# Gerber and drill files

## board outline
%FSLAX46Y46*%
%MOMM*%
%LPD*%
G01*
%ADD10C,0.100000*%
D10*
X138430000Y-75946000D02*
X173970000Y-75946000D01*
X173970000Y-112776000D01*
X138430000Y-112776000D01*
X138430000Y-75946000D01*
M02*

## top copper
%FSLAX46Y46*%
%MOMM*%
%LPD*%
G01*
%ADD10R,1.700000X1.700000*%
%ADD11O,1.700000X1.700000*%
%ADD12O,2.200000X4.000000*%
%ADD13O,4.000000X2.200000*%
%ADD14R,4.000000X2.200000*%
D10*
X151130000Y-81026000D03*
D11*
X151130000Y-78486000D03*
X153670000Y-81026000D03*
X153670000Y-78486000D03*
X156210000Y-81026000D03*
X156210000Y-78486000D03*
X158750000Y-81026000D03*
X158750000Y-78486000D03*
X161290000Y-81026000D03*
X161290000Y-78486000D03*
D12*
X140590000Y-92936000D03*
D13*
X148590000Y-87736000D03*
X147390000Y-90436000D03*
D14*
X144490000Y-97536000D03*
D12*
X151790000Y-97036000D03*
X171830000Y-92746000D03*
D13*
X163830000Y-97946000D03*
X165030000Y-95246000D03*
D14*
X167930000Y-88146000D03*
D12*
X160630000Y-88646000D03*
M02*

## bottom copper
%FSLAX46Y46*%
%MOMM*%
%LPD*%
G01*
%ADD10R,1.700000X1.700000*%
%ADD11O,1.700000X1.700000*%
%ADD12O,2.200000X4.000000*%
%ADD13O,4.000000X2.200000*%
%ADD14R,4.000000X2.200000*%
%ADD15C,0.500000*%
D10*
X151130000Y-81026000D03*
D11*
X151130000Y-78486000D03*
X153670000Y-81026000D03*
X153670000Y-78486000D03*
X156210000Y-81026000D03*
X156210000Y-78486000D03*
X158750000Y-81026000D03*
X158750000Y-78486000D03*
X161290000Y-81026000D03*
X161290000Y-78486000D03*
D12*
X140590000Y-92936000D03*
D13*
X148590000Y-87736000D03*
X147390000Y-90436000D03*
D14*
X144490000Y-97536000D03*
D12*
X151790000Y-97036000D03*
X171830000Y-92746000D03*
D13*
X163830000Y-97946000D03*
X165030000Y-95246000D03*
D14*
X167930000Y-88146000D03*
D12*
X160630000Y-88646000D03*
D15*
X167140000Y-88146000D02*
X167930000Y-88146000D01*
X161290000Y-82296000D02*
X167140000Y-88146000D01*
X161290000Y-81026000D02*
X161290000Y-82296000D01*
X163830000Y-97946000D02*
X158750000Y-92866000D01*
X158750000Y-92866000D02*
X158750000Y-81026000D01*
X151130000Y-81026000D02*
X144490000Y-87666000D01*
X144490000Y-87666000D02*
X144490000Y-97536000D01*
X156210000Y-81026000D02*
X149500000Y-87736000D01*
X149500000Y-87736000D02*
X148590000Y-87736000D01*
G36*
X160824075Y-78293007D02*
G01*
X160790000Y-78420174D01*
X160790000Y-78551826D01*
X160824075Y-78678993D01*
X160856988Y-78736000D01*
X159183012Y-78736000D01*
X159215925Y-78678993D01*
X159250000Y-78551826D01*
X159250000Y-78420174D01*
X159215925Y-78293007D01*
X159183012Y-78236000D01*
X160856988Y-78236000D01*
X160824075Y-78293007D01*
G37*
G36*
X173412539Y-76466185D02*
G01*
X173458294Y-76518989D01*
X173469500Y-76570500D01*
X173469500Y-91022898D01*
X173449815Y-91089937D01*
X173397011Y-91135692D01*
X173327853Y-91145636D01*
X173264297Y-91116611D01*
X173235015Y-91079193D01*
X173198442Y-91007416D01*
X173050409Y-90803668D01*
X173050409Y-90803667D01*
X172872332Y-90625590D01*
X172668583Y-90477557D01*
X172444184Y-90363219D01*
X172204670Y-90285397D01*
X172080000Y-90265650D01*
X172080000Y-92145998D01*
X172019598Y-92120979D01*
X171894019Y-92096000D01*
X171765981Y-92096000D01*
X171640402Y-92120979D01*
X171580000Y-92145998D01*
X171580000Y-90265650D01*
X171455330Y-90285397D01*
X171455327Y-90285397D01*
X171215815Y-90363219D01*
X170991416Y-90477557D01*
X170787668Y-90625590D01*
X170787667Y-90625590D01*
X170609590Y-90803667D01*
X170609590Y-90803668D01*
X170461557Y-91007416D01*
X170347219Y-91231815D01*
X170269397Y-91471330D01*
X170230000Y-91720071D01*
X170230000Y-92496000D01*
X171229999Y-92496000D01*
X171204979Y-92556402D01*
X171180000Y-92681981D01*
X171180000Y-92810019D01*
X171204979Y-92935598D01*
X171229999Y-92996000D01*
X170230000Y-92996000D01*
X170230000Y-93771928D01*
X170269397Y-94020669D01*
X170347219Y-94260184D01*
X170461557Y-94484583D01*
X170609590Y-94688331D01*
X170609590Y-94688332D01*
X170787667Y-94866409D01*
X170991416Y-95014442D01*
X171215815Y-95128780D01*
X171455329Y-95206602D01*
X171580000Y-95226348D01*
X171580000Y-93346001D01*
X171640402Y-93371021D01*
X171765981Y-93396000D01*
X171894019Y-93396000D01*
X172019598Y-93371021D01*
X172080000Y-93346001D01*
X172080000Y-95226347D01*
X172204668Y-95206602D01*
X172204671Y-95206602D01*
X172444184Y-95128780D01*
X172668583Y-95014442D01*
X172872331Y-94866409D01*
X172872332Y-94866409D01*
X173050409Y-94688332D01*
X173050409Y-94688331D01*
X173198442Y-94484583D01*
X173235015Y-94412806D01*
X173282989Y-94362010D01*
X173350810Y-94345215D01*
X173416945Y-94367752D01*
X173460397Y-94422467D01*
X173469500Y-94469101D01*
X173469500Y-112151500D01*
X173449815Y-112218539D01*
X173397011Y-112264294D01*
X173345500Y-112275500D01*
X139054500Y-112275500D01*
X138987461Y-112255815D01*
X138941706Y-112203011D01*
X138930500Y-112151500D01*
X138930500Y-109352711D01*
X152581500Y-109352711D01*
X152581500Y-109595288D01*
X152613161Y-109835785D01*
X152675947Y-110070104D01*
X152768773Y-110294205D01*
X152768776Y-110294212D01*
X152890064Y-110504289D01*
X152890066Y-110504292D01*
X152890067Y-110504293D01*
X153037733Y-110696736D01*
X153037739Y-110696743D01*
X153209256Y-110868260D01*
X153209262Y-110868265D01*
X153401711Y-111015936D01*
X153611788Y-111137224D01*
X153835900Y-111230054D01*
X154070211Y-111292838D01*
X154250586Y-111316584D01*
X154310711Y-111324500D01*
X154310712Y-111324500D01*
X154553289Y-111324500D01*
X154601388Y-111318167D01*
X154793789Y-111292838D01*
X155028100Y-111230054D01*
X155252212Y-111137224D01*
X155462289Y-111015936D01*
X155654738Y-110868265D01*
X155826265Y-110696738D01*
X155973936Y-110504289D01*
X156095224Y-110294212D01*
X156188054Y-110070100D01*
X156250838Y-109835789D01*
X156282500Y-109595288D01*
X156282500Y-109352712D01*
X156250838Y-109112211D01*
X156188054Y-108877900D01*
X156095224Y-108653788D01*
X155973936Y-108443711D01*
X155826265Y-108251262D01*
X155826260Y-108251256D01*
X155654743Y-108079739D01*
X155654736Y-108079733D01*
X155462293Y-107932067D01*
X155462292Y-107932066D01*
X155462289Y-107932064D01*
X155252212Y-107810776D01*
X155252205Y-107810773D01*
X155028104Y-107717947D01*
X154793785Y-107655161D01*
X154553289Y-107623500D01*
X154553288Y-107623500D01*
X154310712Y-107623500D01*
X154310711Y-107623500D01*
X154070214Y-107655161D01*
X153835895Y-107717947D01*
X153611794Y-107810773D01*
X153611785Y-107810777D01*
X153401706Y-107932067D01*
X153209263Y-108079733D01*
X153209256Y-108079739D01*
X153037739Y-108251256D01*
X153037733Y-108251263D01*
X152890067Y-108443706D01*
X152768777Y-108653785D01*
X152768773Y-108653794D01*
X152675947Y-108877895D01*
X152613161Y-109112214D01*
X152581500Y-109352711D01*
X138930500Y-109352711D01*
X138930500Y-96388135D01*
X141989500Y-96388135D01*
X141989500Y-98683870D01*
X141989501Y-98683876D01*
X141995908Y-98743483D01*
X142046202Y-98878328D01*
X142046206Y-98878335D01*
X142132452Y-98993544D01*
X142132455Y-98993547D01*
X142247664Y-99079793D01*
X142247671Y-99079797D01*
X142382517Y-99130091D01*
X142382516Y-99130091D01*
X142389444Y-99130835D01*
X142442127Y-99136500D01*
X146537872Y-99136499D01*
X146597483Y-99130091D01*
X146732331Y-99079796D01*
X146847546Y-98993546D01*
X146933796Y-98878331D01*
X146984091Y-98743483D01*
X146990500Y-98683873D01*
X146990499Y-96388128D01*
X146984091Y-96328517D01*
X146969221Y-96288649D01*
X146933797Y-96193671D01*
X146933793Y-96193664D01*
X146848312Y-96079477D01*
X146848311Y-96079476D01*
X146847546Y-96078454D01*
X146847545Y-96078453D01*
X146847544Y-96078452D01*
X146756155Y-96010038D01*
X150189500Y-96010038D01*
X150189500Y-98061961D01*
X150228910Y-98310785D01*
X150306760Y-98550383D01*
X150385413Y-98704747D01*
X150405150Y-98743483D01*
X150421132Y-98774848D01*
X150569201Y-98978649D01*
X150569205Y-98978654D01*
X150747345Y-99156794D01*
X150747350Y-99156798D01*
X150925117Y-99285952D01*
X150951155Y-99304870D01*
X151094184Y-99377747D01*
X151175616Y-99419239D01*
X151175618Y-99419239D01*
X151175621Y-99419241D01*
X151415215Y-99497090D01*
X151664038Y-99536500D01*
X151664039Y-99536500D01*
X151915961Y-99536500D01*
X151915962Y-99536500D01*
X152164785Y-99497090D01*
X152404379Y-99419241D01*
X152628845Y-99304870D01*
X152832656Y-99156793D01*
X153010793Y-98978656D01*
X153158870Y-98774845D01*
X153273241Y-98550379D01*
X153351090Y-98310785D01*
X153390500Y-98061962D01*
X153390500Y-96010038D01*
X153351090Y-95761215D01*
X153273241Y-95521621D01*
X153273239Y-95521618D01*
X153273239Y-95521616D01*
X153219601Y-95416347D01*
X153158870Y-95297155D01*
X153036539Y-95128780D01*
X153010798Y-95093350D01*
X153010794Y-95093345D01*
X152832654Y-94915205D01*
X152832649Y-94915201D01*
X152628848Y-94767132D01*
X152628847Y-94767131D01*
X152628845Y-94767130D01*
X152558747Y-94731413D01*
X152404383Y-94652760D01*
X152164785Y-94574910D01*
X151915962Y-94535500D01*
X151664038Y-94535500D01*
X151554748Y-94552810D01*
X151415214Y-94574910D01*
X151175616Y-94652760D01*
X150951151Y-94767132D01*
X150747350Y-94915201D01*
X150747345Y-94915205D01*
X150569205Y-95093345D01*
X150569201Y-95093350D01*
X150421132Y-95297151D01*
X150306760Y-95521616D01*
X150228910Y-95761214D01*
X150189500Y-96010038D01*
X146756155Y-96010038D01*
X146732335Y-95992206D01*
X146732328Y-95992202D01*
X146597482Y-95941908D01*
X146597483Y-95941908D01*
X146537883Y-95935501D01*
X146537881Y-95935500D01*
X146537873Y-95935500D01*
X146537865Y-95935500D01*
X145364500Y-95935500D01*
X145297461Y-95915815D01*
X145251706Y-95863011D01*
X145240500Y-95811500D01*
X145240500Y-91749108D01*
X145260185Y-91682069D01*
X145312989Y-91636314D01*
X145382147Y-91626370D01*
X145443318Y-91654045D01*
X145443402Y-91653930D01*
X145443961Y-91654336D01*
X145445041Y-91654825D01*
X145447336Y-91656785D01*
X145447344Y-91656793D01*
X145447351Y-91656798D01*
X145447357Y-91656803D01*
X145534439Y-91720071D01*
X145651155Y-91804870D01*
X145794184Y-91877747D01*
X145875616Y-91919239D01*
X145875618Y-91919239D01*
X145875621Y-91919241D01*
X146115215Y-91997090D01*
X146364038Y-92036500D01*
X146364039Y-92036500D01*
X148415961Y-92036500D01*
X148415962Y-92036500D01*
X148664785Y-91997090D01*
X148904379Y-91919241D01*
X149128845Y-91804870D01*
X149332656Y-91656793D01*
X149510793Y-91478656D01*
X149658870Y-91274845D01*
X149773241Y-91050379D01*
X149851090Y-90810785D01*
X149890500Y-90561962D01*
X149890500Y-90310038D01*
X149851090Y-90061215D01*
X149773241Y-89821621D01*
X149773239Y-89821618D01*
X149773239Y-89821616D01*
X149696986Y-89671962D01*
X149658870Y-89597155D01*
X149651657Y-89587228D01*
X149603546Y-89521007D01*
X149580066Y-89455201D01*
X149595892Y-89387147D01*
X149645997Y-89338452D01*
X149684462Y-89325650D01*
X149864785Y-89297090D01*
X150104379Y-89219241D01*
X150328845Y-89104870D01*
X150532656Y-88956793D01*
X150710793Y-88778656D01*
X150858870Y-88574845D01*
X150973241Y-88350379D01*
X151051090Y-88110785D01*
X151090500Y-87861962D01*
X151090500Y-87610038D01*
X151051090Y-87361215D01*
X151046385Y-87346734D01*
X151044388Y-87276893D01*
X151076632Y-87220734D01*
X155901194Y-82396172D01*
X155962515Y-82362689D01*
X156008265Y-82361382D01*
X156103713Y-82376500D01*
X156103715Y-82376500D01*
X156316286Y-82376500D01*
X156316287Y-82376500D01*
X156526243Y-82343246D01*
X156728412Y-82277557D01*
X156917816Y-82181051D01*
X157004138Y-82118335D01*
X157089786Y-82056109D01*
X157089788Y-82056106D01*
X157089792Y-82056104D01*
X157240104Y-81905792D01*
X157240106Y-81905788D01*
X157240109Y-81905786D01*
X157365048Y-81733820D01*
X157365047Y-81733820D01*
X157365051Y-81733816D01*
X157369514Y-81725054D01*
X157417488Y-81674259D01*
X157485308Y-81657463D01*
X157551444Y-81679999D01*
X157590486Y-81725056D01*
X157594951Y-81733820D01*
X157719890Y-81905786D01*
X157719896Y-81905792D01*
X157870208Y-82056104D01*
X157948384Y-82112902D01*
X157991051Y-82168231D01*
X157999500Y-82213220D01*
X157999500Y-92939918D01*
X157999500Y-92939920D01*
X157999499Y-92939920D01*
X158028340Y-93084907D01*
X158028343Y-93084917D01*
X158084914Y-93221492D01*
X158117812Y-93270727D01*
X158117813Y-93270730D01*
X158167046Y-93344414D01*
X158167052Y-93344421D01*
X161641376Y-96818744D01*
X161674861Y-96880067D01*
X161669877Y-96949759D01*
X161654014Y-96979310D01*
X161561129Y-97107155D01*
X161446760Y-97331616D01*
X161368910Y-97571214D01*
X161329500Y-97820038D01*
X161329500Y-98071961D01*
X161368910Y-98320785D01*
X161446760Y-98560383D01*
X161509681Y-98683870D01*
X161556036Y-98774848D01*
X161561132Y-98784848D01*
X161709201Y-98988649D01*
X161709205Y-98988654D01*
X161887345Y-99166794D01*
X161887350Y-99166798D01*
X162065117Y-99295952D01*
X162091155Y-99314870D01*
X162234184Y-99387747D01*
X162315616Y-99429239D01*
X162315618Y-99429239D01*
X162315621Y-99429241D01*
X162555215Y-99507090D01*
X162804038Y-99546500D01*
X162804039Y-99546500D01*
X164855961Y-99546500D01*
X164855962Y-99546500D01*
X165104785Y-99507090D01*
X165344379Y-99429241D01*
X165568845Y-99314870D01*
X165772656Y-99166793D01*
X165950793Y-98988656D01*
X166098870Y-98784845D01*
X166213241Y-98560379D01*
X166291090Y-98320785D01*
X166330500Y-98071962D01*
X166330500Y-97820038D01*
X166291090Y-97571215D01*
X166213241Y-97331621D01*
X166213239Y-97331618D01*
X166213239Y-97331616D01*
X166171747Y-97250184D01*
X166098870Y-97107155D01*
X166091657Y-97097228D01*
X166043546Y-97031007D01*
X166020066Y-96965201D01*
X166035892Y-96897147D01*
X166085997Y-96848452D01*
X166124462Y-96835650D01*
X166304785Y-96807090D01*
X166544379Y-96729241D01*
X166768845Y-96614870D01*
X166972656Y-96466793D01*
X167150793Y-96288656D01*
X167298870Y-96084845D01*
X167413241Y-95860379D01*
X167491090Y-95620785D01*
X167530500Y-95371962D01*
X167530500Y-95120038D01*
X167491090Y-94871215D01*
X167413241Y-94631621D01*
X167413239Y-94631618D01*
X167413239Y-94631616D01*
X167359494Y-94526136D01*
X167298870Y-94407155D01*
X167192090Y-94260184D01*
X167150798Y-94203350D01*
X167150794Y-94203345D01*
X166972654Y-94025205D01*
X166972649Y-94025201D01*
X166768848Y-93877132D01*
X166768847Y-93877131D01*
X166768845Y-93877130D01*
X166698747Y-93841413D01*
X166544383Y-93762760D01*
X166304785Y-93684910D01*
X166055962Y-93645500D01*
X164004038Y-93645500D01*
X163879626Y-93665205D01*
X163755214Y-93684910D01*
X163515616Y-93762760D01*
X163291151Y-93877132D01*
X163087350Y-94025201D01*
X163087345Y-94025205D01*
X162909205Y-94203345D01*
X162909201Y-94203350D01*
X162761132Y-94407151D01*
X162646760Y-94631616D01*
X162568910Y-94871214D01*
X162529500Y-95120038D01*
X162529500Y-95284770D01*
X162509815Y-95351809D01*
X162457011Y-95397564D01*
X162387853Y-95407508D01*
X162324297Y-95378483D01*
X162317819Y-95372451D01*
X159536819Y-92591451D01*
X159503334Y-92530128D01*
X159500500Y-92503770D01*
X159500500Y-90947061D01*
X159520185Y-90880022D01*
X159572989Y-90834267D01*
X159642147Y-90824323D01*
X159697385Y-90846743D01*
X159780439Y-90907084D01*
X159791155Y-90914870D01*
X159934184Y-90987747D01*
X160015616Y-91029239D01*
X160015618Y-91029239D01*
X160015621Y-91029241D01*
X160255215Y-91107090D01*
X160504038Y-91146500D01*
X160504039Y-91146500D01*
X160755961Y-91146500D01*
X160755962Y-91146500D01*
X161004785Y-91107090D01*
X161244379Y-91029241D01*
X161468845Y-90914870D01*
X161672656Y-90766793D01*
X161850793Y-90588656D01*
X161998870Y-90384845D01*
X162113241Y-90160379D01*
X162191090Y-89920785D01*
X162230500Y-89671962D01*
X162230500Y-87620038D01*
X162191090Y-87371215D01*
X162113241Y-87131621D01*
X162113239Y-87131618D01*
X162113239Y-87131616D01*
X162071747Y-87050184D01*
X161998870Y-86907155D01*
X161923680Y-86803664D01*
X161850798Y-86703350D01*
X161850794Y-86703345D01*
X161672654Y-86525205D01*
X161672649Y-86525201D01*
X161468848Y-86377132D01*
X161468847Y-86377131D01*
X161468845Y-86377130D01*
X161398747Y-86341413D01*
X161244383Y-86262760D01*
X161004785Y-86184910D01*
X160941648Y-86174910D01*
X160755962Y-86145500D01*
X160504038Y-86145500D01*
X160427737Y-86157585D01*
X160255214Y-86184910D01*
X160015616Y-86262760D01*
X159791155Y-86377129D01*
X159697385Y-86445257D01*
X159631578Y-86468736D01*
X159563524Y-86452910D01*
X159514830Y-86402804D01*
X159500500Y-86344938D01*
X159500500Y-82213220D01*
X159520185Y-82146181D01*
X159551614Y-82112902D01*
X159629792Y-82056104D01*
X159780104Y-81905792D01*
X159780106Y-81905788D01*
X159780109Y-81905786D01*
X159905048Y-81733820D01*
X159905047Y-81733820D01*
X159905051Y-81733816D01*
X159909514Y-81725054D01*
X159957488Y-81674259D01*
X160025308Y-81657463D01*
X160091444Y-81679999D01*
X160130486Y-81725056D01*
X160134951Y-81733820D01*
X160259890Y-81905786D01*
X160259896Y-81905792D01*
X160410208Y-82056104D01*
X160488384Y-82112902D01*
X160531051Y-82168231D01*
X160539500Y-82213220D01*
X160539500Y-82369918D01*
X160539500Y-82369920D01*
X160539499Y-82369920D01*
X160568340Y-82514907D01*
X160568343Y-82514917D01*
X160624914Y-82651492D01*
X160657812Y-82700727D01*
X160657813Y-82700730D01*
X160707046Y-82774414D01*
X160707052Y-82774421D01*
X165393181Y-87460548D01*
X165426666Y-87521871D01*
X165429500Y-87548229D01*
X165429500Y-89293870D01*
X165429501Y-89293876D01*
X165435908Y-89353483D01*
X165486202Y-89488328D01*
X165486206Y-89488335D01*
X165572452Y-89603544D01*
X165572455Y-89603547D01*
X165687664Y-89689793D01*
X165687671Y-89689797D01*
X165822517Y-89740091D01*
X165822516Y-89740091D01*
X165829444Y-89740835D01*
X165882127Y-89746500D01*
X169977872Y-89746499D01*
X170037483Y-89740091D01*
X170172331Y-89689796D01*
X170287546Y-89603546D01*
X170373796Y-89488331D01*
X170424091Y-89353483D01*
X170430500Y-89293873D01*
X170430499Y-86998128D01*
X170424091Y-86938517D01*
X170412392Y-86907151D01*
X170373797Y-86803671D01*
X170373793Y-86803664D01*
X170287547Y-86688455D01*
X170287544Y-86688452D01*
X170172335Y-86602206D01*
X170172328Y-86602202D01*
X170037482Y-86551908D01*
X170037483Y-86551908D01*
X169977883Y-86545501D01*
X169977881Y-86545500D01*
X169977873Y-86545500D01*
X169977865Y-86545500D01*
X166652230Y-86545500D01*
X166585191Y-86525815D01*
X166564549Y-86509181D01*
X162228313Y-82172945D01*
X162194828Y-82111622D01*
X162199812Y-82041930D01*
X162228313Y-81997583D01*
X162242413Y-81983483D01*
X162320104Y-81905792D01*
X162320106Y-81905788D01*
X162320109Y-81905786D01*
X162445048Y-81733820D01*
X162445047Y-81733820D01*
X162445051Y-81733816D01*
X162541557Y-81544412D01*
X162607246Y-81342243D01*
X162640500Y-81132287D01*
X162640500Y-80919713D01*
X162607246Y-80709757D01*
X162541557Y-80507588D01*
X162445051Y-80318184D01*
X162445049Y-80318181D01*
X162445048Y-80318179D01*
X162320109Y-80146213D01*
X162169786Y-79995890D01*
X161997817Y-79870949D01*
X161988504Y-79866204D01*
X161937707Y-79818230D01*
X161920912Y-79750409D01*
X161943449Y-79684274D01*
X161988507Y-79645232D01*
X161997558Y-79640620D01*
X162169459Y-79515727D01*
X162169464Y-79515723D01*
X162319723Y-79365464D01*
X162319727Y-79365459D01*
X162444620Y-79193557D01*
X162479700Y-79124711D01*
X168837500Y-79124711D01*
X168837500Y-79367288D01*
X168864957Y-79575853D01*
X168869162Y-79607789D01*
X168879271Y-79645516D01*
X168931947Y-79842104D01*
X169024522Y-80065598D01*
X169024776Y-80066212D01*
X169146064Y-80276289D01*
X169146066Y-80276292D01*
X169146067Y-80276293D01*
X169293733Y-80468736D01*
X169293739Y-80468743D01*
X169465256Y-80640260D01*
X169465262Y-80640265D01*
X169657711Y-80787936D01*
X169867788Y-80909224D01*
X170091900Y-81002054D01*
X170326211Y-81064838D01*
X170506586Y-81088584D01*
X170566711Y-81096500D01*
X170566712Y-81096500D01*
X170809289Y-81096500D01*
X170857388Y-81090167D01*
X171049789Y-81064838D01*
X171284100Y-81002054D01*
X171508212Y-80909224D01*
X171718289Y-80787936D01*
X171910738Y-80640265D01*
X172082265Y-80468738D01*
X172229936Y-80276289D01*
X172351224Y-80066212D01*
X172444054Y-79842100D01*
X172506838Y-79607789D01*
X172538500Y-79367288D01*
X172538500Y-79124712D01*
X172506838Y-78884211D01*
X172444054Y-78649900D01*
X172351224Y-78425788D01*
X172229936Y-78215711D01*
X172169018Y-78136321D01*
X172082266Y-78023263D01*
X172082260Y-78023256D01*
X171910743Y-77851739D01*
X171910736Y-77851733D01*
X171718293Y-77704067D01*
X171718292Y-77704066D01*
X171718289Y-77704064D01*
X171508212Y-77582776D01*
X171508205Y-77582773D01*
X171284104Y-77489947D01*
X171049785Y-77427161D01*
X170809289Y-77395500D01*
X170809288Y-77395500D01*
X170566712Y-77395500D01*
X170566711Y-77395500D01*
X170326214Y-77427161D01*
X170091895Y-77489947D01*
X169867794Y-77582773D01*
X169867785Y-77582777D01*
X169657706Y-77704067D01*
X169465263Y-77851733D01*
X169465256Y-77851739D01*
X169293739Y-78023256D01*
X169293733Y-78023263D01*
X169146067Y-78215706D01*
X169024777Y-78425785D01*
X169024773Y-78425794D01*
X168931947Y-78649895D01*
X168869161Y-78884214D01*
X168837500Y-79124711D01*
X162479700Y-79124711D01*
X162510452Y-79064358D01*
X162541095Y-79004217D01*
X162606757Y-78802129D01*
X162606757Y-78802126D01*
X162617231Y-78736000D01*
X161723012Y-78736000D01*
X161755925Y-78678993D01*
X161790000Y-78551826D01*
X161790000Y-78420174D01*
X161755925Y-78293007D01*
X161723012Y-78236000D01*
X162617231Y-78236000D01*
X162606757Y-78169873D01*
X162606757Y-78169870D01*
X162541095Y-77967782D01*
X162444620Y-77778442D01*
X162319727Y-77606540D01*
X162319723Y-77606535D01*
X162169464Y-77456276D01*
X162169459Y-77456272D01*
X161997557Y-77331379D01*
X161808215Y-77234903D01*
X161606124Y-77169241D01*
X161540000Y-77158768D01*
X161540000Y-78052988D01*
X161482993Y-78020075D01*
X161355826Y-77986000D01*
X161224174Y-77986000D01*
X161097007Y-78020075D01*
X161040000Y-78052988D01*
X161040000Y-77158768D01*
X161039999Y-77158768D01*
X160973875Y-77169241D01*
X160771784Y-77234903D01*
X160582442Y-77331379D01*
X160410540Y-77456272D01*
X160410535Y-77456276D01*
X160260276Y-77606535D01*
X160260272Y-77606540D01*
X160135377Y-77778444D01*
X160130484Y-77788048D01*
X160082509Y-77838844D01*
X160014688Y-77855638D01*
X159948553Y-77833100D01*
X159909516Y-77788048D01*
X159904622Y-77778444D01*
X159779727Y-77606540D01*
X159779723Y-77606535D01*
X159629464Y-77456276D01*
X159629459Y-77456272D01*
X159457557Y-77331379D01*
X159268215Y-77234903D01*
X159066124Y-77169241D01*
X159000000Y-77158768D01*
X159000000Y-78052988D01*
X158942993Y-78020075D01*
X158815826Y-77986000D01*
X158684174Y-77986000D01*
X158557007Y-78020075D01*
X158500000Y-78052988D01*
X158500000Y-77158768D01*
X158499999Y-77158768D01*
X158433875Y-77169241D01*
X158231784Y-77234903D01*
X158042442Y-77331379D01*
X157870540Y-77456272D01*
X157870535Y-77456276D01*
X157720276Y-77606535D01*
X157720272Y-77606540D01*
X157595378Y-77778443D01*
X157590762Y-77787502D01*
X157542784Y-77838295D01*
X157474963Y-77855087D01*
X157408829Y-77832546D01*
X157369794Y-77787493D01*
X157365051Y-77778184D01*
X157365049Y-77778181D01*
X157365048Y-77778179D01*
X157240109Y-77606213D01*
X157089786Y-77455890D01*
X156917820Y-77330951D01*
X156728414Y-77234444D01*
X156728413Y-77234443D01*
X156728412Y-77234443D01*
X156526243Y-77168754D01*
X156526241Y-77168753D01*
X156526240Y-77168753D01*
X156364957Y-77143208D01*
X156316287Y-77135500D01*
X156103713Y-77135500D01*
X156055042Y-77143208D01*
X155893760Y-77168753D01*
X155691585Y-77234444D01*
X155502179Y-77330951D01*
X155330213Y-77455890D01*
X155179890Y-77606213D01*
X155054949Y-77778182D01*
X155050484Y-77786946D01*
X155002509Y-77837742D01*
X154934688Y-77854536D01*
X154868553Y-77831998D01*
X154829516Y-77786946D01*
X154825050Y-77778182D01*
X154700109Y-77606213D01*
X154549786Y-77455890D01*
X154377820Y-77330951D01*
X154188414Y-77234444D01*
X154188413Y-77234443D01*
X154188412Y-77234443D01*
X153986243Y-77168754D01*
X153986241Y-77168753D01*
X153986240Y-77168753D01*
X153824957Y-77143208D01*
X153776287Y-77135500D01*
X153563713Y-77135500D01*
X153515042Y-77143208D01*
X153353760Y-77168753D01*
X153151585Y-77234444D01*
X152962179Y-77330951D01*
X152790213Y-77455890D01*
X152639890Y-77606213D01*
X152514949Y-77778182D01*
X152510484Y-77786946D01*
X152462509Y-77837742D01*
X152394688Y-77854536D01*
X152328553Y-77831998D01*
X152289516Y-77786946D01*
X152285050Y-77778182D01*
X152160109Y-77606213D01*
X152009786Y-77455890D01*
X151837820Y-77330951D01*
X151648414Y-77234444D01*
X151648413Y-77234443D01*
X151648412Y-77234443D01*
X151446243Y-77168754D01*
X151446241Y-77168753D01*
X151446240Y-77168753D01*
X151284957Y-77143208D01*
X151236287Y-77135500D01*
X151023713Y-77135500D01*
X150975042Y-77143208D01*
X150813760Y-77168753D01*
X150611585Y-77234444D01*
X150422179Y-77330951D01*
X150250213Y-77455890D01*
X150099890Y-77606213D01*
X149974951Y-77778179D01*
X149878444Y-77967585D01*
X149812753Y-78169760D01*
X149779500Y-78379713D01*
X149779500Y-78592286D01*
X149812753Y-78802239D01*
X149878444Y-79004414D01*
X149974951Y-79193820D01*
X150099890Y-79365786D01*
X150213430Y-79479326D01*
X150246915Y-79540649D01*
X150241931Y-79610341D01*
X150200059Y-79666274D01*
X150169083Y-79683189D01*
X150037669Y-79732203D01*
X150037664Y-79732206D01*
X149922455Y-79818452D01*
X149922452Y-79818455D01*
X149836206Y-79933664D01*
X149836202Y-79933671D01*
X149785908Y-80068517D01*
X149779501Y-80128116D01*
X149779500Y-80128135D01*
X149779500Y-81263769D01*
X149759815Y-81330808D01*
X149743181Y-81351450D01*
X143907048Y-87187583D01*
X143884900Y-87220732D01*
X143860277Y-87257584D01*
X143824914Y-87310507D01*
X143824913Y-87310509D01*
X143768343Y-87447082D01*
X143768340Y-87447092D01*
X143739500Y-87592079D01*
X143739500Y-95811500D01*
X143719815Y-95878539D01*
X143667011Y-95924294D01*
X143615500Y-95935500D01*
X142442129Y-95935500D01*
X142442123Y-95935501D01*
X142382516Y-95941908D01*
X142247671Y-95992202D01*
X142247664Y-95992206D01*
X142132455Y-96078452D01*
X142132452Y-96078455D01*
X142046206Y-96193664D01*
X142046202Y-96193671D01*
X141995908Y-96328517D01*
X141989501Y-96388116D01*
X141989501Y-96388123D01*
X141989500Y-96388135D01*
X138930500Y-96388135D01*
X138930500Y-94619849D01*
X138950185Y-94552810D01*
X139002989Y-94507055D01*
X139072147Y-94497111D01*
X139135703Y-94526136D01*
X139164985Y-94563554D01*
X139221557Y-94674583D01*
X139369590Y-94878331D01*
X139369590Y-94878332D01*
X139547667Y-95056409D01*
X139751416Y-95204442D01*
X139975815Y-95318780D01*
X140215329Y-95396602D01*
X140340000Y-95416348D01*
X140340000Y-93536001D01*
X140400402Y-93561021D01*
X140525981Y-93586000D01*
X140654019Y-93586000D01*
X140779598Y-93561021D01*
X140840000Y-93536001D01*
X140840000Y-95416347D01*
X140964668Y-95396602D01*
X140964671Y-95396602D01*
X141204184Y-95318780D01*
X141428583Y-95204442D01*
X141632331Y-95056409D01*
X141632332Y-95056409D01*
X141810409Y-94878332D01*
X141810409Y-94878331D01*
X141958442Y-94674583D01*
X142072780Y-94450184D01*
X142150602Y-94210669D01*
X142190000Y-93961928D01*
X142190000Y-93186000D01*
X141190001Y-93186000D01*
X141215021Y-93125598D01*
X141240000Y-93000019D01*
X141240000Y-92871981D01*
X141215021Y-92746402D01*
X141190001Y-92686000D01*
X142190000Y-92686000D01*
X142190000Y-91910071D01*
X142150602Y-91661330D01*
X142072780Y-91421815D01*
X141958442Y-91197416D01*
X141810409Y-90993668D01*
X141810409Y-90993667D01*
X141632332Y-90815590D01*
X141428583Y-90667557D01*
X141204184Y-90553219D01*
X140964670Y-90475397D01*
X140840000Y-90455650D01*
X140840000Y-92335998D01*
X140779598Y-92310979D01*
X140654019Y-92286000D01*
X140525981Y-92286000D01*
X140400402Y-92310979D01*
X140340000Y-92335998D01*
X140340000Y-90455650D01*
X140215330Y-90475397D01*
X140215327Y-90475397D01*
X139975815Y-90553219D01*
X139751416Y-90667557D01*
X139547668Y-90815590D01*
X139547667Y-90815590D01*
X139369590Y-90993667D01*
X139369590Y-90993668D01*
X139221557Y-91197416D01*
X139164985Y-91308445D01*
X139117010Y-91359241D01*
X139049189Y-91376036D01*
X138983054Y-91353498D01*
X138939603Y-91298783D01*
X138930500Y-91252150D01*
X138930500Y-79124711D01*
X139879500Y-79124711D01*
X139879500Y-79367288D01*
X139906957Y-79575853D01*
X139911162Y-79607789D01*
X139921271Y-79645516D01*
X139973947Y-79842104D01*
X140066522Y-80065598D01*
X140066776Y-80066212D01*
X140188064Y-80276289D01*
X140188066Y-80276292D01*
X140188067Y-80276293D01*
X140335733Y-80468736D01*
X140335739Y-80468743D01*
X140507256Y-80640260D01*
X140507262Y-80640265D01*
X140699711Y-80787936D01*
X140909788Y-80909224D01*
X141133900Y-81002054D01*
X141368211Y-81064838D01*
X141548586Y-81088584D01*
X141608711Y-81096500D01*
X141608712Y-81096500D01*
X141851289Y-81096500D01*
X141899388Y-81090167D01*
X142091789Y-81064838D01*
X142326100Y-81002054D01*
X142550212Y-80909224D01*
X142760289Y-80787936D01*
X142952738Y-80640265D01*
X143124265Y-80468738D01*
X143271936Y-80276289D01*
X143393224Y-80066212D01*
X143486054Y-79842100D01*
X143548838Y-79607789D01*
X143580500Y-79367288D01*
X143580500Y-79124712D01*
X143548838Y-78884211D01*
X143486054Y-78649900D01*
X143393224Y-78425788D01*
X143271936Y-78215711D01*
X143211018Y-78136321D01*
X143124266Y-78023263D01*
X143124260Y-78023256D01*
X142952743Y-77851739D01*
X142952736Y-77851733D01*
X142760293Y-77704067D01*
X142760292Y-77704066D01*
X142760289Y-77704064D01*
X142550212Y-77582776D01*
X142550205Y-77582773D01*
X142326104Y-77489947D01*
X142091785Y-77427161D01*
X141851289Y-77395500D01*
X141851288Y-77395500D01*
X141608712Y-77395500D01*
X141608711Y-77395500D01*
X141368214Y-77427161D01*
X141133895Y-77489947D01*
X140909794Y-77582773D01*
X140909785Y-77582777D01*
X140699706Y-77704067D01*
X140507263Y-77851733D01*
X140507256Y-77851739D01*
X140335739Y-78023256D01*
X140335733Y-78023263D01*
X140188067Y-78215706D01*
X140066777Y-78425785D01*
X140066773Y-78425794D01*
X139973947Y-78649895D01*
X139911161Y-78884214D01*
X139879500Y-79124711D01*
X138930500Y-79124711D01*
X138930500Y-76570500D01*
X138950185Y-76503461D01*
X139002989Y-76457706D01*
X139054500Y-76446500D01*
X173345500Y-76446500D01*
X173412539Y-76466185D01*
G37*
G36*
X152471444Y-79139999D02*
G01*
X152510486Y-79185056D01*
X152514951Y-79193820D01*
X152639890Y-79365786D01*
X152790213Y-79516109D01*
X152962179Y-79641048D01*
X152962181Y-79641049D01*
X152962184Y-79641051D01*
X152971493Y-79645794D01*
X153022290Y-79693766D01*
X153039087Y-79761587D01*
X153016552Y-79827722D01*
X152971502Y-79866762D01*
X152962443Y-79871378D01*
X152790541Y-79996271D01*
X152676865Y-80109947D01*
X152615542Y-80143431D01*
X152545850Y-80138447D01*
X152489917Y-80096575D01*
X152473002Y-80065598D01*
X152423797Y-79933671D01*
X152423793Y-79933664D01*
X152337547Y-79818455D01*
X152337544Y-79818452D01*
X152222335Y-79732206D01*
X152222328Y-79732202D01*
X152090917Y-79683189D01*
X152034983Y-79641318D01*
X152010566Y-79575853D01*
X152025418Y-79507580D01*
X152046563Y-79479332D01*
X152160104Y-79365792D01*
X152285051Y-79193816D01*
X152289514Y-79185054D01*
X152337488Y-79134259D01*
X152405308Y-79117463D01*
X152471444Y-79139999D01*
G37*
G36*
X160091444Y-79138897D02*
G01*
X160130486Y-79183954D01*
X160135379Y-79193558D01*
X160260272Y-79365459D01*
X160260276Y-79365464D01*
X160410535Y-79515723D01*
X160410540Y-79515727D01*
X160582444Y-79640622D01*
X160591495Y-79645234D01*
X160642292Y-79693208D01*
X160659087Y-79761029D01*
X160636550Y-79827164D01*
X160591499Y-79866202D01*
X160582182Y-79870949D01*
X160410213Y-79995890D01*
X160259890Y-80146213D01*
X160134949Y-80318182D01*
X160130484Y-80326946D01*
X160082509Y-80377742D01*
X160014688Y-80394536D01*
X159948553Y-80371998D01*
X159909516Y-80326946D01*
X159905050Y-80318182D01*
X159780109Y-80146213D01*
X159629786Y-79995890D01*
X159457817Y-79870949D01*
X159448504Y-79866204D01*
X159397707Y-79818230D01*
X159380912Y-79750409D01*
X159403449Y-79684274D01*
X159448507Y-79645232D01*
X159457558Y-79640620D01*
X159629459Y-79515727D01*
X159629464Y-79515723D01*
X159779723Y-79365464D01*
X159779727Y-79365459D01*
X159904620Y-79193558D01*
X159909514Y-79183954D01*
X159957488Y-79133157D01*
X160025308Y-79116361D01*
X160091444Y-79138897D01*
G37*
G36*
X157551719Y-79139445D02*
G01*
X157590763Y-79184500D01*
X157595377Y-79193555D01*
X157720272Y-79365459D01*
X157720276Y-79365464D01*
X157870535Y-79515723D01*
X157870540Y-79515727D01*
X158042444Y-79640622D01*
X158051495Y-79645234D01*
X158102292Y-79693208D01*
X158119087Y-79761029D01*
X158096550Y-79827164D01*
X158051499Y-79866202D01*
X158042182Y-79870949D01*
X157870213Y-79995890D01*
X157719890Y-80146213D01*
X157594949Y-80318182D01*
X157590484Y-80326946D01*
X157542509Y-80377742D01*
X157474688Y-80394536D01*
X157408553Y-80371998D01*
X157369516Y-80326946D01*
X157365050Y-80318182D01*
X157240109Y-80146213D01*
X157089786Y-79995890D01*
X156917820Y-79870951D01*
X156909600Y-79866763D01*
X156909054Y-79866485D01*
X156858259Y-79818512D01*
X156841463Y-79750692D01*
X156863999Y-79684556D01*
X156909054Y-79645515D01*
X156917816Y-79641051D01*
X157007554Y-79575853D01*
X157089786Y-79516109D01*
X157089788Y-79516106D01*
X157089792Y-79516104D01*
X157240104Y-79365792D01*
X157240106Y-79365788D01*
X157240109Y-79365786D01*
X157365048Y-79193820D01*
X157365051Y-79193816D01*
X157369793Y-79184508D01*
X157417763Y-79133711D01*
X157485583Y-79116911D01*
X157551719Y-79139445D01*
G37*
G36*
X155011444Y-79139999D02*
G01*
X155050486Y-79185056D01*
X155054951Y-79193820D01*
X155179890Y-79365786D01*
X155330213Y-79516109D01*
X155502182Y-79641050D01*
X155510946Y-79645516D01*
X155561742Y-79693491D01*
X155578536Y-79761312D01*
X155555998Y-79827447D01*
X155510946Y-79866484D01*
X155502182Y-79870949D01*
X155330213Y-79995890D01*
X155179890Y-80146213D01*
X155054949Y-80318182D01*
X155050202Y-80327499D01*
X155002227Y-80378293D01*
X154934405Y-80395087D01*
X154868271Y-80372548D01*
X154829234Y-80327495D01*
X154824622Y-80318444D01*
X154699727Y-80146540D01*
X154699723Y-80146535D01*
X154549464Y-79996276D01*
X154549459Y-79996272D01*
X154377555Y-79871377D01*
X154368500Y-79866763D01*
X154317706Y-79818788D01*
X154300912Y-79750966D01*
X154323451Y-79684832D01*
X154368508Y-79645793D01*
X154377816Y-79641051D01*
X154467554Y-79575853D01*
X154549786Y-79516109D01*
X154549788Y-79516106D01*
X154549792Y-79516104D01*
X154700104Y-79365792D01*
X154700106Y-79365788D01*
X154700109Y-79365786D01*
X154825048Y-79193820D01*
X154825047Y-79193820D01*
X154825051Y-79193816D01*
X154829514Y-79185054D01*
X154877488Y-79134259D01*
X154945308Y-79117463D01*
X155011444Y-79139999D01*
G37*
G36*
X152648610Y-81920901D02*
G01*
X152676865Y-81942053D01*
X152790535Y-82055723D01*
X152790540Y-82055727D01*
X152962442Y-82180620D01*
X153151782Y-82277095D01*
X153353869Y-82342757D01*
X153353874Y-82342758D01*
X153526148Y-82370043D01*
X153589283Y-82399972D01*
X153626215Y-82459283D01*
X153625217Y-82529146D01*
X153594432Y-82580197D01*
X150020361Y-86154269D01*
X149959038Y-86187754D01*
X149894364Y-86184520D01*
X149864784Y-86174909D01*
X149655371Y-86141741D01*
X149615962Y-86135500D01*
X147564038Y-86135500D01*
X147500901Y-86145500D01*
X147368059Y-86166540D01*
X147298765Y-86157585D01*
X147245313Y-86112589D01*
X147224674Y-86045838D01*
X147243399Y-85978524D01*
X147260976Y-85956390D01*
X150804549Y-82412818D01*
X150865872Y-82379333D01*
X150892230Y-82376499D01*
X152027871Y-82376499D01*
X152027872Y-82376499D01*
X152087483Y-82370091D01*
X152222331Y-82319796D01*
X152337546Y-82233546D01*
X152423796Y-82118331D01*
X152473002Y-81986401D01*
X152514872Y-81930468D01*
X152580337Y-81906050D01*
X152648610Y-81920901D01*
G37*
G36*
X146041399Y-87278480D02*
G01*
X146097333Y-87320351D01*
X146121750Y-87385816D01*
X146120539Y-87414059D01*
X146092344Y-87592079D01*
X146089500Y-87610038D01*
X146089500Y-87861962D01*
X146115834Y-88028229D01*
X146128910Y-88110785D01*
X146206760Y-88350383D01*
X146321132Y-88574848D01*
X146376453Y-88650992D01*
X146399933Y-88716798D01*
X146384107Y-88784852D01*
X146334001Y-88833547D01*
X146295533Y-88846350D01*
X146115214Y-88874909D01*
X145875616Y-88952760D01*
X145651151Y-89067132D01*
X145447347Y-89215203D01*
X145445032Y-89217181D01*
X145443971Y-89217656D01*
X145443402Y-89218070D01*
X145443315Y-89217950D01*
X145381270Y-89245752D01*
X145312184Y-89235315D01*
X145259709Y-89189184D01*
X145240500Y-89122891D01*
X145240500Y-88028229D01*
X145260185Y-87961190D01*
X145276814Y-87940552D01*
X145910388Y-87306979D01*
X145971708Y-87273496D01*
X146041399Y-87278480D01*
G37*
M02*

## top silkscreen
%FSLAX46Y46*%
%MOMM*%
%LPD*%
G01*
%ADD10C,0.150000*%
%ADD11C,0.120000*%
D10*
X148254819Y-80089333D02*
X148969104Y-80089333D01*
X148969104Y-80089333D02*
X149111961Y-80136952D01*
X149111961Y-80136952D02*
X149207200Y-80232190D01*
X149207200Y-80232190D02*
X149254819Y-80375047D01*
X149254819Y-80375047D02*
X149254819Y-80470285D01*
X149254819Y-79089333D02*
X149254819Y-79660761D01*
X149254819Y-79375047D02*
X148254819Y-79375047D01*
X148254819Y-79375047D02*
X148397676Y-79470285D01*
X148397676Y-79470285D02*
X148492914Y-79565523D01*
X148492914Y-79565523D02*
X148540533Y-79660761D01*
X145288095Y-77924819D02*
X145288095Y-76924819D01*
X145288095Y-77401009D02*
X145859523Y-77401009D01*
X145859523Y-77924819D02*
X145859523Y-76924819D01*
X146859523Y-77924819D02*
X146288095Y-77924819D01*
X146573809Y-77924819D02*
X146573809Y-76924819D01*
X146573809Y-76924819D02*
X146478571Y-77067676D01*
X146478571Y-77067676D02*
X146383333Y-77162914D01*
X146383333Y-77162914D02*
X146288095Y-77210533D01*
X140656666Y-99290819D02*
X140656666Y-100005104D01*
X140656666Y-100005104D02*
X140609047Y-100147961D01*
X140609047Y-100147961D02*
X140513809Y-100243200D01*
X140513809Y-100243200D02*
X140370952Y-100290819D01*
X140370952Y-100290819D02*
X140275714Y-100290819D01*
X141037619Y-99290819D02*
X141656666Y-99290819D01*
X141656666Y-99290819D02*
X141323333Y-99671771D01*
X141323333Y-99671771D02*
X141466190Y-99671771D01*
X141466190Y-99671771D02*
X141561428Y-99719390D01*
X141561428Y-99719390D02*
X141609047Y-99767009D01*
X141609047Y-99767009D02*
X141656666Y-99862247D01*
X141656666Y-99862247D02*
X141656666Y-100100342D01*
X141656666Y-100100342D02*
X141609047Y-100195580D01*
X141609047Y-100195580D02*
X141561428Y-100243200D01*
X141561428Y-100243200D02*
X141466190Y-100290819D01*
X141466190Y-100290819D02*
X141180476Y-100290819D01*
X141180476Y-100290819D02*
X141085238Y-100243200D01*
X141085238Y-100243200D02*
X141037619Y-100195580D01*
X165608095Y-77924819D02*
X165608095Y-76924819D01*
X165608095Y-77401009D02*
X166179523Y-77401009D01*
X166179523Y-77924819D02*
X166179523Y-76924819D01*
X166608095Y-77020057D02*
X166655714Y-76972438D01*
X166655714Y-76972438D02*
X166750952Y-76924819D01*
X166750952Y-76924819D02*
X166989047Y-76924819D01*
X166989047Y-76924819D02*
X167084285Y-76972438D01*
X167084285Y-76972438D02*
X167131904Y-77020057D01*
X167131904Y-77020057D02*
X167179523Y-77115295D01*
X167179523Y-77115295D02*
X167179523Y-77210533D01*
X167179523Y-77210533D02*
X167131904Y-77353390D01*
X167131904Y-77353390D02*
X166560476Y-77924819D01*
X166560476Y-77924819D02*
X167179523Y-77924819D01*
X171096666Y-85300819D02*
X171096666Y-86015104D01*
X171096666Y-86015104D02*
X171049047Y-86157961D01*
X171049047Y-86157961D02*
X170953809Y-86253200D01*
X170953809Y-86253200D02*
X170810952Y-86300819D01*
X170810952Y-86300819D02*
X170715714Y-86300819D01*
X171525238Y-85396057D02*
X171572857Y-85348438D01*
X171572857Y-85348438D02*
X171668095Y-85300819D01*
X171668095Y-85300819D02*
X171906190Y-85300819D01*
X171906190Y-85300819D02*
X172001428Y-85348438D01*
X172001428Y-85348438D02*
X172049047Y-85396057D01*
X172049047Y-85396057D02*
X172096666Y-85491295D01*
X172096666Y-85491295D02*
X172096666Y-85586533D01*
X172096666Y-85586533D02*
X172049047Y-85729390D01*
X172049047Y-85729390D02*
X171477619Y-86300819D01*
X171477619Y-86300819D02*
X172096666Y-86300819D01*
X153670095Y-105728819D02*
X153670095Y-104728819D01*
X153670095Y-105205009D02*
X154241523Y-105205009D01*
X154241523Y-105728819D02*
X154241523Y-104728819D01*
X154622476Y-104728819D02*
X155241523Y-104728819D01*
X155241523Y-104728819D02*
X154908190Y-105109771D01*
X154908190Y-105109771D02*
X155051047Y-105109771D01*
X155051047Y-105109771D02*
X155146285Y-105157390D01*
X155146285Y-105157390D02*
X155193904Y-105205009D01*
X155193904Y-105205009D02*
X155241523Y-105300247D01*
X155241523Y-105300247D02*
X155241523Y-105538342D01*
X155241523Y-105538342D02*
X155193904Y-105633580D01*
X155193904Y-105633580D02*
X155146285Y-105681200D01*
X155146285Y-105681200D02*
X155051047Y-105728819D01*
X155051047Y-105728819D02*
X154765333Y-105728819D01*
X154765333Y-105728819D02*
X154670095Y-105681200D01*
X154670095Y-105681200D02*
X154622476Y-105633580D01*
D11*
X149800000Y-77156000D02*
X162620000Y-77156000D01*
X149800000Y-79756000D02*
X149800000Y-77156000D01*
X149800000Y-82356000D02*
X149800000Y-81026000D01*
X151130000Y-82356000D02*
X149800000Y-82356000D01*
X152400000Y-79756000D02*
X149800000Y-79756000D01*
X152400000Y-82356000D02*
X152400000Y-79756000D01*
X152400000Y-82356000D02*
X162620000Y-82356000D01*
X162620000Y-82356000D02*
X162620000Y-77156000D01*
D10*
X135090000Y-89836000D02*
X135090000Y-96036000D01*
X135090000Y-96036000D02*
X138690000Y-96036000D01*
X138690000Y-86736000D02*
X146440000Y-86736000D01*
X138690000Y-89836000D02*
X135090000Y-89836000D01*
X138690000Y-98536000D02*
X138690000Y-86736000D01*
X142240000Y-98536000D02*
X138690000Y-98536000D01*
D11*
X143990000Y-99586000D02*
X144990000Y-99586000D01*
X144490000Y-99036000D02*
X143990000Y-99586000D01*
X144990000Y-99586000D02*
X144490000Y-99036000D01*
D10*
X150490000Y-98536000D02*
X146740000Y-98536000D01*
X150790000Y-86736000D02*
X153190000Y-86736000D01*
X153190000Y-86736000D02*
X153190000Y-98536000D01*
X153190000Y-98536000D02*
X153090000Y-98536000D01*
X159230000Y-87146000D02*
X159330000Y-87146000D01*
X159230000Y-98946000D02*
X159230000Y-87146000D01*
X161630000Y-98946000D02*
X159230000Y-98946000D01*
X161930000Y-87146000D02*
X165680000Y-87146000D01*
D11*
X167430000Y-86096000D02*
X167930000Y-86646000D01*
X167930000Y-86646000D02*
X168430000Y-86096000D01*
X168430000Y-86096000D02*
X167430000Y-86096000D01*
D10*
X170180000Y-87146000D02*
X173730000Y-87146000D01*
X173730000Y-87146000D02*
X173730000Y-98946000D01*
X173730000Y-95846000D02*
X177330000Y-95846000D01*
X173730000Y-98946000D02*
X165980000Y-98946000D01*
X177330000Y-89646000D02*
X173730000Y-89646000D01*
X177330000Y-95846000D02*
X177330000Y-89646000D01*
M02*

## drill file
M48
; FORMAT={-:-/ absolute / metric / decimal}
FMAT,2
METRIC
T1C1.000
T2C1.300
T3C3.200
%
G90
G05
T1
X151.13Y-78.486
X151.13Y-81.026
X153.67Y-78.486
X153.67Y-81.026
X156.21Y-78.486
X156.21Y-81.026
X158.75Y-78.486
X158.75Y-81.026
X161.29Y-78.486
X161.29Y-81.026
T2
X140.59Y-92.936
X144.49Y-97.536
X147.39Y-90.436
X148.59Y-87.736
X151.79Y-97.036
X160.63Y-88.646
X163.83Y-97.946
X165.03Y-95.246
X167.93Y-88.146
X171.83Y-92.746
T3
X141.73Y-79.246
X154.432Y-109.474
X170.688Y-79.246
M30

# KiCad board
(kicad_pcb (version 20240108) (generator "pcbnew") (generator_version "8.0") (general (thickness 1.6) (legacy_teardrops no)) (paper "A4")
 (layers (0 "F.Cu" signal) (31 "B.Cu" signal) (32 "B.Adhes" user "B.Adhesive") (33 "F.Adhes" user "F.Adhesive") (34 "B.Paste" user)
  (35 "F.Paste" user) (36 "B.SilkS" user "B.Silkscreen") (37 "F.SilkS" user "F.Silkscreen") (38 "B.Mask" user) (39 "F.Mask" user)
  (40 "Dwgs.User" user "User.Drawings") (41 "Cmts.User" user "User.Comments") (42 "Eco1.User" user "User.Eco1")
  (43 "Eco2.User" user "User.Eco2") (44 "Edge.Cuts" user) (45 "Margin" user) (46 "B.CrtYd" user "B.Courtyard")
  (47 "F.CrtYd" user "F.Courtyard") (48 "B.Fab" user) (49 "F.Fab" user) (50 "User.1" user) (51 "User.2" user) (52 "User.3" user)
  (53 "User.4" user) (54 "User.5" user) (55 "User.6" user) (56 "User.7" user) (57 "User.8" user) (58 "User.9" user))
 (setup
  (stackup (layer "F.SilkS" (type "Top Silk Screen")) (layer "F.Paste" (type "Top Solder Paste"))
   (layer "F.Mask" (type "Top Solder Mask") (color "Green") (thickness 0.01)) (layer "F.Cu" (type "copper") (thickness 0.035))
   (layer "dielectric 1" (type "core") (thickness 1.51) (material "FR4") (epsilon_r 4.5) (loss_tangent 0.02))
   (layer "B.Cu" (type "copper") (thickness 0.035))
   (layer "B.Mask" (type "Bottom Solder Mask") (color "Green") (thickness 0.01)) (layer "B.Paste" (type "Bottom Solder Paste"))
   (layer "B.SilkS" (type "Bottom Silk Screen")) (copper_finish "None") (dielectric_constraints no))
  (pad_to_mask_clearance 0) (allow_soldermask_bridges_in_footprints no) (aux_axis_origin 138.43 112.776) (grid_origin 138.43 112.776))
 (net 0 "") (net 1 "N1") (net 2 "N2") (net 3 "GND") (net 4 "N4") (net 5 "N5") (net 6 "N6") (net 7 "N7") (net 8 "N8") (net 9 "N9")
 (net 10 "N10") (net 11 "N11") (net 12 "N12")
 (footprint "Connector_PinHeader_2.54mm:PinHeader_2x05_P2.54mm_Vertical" (layer "F.Cu") (at 151.13 81.026 90)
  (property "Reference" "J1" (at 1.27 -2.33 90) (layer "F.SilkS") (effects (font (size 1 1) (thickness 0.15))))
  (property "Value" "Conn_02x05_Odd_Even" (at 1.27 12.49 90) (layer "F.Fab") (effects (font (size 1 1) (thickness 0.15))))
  (fp_line (start 3.87 -1.33) (end 3.87 11.49) (stroke (width 0.12) (type solid)) (layer "F.SilkS"))
  (fp_line (start 1.27 -1.33) (end 3.87 -1.33) (stroke (width 0.12) (type solid)) (layer "F.SilkS"))
  (fp_line (start -1.33 -1.33) (end 0 -1.33) (stroke (width 0.12) (type solid)) (layer "F.SilkS"))
  (fp_line (start -1.33 0) (end -1.33 -1.33) (stroke (width 0.12) (type solid)) (layer "F.SilkS"))
  (fp_line (start 1.27 1.27) (end 1.27 -1.33) (stroke (width 0.12) (type solid)) (layer "F.SilkS"))
  (fp_line (start -1.33 1.27) (end 1.27 1.27) (stroke (width 0.12) (type solid)) (layer "F.SilkS"))
  (fp_line (start -1.33 1.27) (end -1.33 11.49) (stroke (width 0.12) (type solid)) (layer "F.SilkS"))
  (fp_line (start -1.33 11.49) (end 3.87 11.49) (stroke (width 0.12) (type solid)) (layer "F.SilkS"))
  (pad "1" thru_hole rect (at 0 0 90) (size 1.7 1.7) (drill 1) (layers "*.Cu" "*.Mask") (remove_unused_layers no) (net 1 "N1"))
  (pad "2" thru_hole oval (at 2.54 0 90) (size 1.7 1.7) (drill 1) (layers "*.Cu" "*.Mask") (remove_unused_layers no) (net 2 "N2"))
  (pad "3" thru_hole oval (at 0 2.54 90) (size 1.7 1.7) (drill 1) (layers "*.Cu" "*.Mask") (remove_unused_layers no) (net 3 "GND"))
  (pad "4" thru_hole oval (at 2.54 2.54 90) (size 1.7 1.7) (drill 1) (layers "*.Cu" "*.Mask") (remove_unused_layers no) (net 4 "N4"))
  (pad "5" thru_hole oval (at 0 5.08 90) (size 1.7 1.7) (drill 1) (layers "*.Cu" "*.Mask") (remove_unused_layers no) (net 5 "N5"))
  (pad "6" thru_hole oval (at 2.54 5.08 90) (size 1.7 1.7) (drill 1) (layers "*.Cu" "*.Mask") (remove_unused_layers no) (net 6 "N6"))
  (pad "7" thru_hole oval (at 0 7.62 90) (size 1.7 1.7) (drill 1) (layers "*.Cu" "*.Mask") (remove_unused_layers no) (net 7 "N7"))
  (pad "8" thru_hole oval (at 2.54 7.62 90) (size 1.7 1.7) (drill 1) (layers "*.Cu" "*.Mask") (remove_unused_layers no) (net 3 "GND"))
  (pad "9" thru_hole oval (at 0 10.16 90) (size 1.7 1.7) (drill 1) (layers "*.Cu" "*.Mask") (remove_unused_layers no) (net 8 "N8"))
  (pad "10" thru_hole oval (at 2.54 10.16 90) (size 1.7 1.7) (drill 1) (layers "*.Cu" "*.Mask") (remove_unused_layers no) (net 3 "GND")))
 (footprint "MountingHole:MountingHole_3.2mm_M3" (layer "F.Cu") (at 141.73 79.246)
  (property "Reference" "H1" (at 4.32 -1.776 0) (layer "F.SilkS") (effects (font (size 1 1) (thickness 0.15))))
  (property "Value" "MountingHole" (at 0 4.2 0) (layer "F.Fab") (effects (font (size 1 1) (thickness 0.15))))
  (pad "" np_thru_hole circle (at 0 0) (size 3.2 3.2) (drill 3.2) (layers "*.Cu" "*.Mask")))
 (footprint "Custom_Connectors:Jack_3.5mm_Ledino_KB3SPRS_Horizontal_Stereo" (layer "F.Cu") (at 144.49 97.536)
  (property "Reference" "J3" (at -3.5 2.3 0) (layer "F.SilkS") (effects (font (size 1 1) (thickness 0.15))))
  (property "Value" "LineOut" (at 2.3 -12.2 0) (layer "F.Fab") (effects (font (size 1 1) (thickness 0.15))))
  (fp_line (start -9.4 -7.7) (end -9.4 -1.5) (stroke (width 0.15) (type solid)) (layer "F.SilkS"))
  (fp_line (start -9.4 -1.5) (end -5.8 -1.5) (stroke (width 0.15) (type solid)) (layer "F.SilkS"))
  (fp_line (start -5.8 -10.8) (end 1.95 -10.8) (stroke (width 0.15) (type solid)) (layer "F.SilkS"))
  (fp_line (start -5.8 -7.7) (end -9.4 -7.7) (stroke (width 0.15) (type solid)) (layer "F.SilkS"))
  (fp_line (start -5.8 1) (end -5.8 -10.8) (stroke (width 0.15) (type solid)) (layer "F.SilkS"))
  (fp_line (start -2.25 1) (end -5.8 1) (stroke (width 0.15) (type solid)) (layer "F.SilkS"))
  (fp_line (start -0.5 2.05) (end 0.5 2.05) (stroke (width 0.12) (type solid)) (layer "F.SilkS"))
  (fp_line (start 0 1.5) (end -0.5 2.05) (stroke (width 0.12) (type solid)) (layer "F.SilkS"))
  (fp_line (start 0.5 2.05) (end 0 1.5) (stroke (width 0.12) (type solid)) (layer "F.SilkS"))
  (fp_line (start 6 1) (end 2.25 1) (stroke (width 0.15) (type solid)) (layer "F.SilkS"))
  (fp_line (start 6.3 -10.8) (end 8.7 -10.8) (stroke (width 0.15) (type solid)) (layer "F.SilkS"))
  (fp_line (start 8.7 -10.8) (end 8.7 1) (stroke (width 0.15) (type solid)) (layer "F.SilkS"))
  (fp_line (start 8.7 1) (end 8.6 1) (stroke (width 0.15) (type solid)) (layer "F.SilkS"))
  (pad "G" thru_hole oval (at -3.9 -4.6) (size 2.2 4) (drill 1.3) (layers "*.Cu" "*.Mask" "Eco2.User") (remove_unused_layers no)
   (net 3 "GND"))
  (pad "S" thru_hole oval (at 4.1 -9.8) (size 4 2.2) (drill 1.3) (layers "*.Cu" "*.Mask") (remove_unused_layers no) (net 5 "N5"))
  (pad "SN" thru_hole oval (at 2.9 -7.1) (size 4 2.2) (drill 1.3) (layers "*.Cu" "*.Mask") (remove_unused_layers no) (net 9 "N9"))
  (pad "T" thru_hole rect (at 0 0) (size 4 2.2) (drill 1.3) (layers "*.Cu" "*.Mask") (remove_unused_layers no) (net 1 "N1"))
  (pad "TN" thru_hole oval (at 7.3 -0.5 90) (size 4 2.2) (drill 1.3) (layers "*.Cu" "*.Mask") (remove_unused_layers no) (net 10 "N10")))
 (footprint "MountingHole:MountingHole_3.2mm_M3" (layer "F.Cu") (at 170.688 79.246)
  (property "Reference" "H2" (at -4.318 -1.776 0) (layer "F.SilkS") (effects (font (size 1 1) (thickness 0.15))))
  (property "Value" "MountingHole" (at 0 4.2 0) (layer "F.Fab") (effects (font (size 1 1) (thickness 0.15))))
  (pad "" np_thru_hole circle (at 0 0) (size 3.2 3.2) (drill 3.2) (layers "*.Cu" "*.Mask")))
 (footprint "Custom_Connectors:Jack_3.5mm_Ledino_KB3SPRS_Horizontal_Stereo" (layer "F.Cu") (at 167.93 88.146 180)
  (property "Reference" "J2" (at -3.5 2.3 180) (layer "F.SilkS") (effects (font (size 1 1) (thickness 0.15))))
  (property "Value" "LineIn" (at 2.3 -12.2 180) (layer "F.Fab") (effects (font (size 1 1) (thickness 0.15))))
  (fp_line (start 8.7 1) (end 8.6 1) (stroke (width 0.15) (type solid)) (layer "F.SilkS"))
  (fp_line (start 8.7 -10.8) (end 8.7 1) (stroke (width 0.15) (type solid)) (layer "F.SilkS"))
  (fp_line (start 6.3 -10.8) (end 8.7 -10.8) (stroke (width 0.15) (type solid)) (layer "F.SilkS"))
  (fp_line (start 6 1) (end 2.25 1) (stroke (width 0.15) (type solid)) (layer "F.SilkS"))
  (fp_line (start 0.5 2.05) (end 0 1.5) (stroke (width 0.12) (type solid)) (layer "F.SilkS"))
  (fp_line (start 0 1.5) (end -0.5 2.05) (stroke (width 0.12) (type solid)) (layer "F.SilkS"))
  (fp_line (start -0.5 2.05) (end 0.5 2.05) (stroke (width 0.12) (type solid)) (layer "F.SilkS"))
  (fp_line (start -2.25 1) (end -5.8 1) (stroke (width 0.15) (type solid)) (layer "F.SilkS"))
  (fp_line (start -5.8 1) (end -5.8 -10.8) (stroke (width 0.15) (type solid)) (layer "F.SilkS"))
  (fp_line (start -5.8 -7.7) (end -9.4 -7.7) (stroke (width 0.15) (type solid)) (layer "F.SilkS"))
  (fp_line (start -5.8 -10.8) (end 1.95 -10.8) (stroke (width 0.15) (type solid)) (layer "F.SilkS"))
  (fp_line (start -9.4 -1.5) (end -5.8 -1.5) (stroke (width 0.15) (type solid)) (layer "F.SilkS"))
  (fp_line (start -9.4 -7.7) (end -9.4 -1.5) (stroke (width 0.15) (type solid)) (layer "F.SilkS"))
  (pad "G" thru_hole oval (at -3.9 -4.6 180) (size 2.2 4) (drill 1.3) (layers "*.Cu" "*.Mask" "Eco2.User") (remove_unused_layers no)
   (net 3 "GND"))
  (pad "S" thru_hole oval (at 4.1 -9.8 180) (size 4 2.2) (drill 1.3) (layers "*.Cu" "*.Mask") (remove_unused_layers no) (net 7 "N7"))
  (pad "SN" thru_hole oval (at 2.9 -7.1 180) (size 4 2.2) (drill 1.3) (layers "*.Cu" "*.Mask") (remove_unused_layers no) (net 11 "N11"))
  (pad "T" thru_hole rect (at 0 0 180) (size 4 2.2) (drill 1.3) (layers "*.Cu" "*.Mask") (remove_unused_layers no) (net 8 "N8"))
  (pad "TN" thru_hole oval (at 7.3 -0.5 270) (size 4 2.2) (drill 1.3) (layers "*.Cu" "*.Mask") (remove_unused_layers no) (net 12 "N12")))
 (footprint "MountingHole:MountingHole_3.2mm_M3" (layer "F.Cu") (at 154.432 109.474)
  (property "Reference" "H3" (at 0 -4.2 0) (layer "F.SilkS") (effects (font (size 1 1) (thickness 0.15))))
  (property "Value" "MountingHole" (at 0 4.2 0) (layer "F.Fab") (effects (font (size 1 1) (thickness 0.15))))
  (pad "" np_thru_hole circle (at 0 0) (size 3.2 3.2) (drill 3.2) (layers "*.Cu" "*.Mask")))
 (gr_rect (start 138.43 75.946) (end 173.97 112.776) (stroke (width 0.1) (type default)) (fill none) (layer "Edge.Cuts"))
 (segment (start 167.14 88.146) (end 167.93 88.146) (width 0.5) (layer "B.Cu") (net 8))
 (segment (start 161.29 82.296) (end 167.14 88.146) (width 0.5) (layer "B.Cu") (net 8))
 (segment (start 161.29 81.026) (end 161.29 82.296) (width 0.5) (layer "B.Cu") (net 8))
 (segment (start 163.83 97.946) (end 158.75 92.866) (width 0.5) (layer "B.Cu") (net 7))
 (segment (start 158.75 92.866) (end 158.75 81.026) (width 0.5) (layer "B.Cu") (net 7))
 (segment (start 151.13 81.026) (end 144.49 87.666) (width 0.5) (layer "B.Cu") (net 1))
 (segment (start 144.49 87.666) (end 144.49 97.536) (width 0.5) (layer "B.Cu") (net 1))
 (segment (start 156.21 81.026) (end 149.5 87.736) (width 0.5) (layer "B.Cu") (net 5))
 (segment (start 149.5 87.736) (end 148.59 87.736) (width 0.5) (layer "B.Cu") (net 5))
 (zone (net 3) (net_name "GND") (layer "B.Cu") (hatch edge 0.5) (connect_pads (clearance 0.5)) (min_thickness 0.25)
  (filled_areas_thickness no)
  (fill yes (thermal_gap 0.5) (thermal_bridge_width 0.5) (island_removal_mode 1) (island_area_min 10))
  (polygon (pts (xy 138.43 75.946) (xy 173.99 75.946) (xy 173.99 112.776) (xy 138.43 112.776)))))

